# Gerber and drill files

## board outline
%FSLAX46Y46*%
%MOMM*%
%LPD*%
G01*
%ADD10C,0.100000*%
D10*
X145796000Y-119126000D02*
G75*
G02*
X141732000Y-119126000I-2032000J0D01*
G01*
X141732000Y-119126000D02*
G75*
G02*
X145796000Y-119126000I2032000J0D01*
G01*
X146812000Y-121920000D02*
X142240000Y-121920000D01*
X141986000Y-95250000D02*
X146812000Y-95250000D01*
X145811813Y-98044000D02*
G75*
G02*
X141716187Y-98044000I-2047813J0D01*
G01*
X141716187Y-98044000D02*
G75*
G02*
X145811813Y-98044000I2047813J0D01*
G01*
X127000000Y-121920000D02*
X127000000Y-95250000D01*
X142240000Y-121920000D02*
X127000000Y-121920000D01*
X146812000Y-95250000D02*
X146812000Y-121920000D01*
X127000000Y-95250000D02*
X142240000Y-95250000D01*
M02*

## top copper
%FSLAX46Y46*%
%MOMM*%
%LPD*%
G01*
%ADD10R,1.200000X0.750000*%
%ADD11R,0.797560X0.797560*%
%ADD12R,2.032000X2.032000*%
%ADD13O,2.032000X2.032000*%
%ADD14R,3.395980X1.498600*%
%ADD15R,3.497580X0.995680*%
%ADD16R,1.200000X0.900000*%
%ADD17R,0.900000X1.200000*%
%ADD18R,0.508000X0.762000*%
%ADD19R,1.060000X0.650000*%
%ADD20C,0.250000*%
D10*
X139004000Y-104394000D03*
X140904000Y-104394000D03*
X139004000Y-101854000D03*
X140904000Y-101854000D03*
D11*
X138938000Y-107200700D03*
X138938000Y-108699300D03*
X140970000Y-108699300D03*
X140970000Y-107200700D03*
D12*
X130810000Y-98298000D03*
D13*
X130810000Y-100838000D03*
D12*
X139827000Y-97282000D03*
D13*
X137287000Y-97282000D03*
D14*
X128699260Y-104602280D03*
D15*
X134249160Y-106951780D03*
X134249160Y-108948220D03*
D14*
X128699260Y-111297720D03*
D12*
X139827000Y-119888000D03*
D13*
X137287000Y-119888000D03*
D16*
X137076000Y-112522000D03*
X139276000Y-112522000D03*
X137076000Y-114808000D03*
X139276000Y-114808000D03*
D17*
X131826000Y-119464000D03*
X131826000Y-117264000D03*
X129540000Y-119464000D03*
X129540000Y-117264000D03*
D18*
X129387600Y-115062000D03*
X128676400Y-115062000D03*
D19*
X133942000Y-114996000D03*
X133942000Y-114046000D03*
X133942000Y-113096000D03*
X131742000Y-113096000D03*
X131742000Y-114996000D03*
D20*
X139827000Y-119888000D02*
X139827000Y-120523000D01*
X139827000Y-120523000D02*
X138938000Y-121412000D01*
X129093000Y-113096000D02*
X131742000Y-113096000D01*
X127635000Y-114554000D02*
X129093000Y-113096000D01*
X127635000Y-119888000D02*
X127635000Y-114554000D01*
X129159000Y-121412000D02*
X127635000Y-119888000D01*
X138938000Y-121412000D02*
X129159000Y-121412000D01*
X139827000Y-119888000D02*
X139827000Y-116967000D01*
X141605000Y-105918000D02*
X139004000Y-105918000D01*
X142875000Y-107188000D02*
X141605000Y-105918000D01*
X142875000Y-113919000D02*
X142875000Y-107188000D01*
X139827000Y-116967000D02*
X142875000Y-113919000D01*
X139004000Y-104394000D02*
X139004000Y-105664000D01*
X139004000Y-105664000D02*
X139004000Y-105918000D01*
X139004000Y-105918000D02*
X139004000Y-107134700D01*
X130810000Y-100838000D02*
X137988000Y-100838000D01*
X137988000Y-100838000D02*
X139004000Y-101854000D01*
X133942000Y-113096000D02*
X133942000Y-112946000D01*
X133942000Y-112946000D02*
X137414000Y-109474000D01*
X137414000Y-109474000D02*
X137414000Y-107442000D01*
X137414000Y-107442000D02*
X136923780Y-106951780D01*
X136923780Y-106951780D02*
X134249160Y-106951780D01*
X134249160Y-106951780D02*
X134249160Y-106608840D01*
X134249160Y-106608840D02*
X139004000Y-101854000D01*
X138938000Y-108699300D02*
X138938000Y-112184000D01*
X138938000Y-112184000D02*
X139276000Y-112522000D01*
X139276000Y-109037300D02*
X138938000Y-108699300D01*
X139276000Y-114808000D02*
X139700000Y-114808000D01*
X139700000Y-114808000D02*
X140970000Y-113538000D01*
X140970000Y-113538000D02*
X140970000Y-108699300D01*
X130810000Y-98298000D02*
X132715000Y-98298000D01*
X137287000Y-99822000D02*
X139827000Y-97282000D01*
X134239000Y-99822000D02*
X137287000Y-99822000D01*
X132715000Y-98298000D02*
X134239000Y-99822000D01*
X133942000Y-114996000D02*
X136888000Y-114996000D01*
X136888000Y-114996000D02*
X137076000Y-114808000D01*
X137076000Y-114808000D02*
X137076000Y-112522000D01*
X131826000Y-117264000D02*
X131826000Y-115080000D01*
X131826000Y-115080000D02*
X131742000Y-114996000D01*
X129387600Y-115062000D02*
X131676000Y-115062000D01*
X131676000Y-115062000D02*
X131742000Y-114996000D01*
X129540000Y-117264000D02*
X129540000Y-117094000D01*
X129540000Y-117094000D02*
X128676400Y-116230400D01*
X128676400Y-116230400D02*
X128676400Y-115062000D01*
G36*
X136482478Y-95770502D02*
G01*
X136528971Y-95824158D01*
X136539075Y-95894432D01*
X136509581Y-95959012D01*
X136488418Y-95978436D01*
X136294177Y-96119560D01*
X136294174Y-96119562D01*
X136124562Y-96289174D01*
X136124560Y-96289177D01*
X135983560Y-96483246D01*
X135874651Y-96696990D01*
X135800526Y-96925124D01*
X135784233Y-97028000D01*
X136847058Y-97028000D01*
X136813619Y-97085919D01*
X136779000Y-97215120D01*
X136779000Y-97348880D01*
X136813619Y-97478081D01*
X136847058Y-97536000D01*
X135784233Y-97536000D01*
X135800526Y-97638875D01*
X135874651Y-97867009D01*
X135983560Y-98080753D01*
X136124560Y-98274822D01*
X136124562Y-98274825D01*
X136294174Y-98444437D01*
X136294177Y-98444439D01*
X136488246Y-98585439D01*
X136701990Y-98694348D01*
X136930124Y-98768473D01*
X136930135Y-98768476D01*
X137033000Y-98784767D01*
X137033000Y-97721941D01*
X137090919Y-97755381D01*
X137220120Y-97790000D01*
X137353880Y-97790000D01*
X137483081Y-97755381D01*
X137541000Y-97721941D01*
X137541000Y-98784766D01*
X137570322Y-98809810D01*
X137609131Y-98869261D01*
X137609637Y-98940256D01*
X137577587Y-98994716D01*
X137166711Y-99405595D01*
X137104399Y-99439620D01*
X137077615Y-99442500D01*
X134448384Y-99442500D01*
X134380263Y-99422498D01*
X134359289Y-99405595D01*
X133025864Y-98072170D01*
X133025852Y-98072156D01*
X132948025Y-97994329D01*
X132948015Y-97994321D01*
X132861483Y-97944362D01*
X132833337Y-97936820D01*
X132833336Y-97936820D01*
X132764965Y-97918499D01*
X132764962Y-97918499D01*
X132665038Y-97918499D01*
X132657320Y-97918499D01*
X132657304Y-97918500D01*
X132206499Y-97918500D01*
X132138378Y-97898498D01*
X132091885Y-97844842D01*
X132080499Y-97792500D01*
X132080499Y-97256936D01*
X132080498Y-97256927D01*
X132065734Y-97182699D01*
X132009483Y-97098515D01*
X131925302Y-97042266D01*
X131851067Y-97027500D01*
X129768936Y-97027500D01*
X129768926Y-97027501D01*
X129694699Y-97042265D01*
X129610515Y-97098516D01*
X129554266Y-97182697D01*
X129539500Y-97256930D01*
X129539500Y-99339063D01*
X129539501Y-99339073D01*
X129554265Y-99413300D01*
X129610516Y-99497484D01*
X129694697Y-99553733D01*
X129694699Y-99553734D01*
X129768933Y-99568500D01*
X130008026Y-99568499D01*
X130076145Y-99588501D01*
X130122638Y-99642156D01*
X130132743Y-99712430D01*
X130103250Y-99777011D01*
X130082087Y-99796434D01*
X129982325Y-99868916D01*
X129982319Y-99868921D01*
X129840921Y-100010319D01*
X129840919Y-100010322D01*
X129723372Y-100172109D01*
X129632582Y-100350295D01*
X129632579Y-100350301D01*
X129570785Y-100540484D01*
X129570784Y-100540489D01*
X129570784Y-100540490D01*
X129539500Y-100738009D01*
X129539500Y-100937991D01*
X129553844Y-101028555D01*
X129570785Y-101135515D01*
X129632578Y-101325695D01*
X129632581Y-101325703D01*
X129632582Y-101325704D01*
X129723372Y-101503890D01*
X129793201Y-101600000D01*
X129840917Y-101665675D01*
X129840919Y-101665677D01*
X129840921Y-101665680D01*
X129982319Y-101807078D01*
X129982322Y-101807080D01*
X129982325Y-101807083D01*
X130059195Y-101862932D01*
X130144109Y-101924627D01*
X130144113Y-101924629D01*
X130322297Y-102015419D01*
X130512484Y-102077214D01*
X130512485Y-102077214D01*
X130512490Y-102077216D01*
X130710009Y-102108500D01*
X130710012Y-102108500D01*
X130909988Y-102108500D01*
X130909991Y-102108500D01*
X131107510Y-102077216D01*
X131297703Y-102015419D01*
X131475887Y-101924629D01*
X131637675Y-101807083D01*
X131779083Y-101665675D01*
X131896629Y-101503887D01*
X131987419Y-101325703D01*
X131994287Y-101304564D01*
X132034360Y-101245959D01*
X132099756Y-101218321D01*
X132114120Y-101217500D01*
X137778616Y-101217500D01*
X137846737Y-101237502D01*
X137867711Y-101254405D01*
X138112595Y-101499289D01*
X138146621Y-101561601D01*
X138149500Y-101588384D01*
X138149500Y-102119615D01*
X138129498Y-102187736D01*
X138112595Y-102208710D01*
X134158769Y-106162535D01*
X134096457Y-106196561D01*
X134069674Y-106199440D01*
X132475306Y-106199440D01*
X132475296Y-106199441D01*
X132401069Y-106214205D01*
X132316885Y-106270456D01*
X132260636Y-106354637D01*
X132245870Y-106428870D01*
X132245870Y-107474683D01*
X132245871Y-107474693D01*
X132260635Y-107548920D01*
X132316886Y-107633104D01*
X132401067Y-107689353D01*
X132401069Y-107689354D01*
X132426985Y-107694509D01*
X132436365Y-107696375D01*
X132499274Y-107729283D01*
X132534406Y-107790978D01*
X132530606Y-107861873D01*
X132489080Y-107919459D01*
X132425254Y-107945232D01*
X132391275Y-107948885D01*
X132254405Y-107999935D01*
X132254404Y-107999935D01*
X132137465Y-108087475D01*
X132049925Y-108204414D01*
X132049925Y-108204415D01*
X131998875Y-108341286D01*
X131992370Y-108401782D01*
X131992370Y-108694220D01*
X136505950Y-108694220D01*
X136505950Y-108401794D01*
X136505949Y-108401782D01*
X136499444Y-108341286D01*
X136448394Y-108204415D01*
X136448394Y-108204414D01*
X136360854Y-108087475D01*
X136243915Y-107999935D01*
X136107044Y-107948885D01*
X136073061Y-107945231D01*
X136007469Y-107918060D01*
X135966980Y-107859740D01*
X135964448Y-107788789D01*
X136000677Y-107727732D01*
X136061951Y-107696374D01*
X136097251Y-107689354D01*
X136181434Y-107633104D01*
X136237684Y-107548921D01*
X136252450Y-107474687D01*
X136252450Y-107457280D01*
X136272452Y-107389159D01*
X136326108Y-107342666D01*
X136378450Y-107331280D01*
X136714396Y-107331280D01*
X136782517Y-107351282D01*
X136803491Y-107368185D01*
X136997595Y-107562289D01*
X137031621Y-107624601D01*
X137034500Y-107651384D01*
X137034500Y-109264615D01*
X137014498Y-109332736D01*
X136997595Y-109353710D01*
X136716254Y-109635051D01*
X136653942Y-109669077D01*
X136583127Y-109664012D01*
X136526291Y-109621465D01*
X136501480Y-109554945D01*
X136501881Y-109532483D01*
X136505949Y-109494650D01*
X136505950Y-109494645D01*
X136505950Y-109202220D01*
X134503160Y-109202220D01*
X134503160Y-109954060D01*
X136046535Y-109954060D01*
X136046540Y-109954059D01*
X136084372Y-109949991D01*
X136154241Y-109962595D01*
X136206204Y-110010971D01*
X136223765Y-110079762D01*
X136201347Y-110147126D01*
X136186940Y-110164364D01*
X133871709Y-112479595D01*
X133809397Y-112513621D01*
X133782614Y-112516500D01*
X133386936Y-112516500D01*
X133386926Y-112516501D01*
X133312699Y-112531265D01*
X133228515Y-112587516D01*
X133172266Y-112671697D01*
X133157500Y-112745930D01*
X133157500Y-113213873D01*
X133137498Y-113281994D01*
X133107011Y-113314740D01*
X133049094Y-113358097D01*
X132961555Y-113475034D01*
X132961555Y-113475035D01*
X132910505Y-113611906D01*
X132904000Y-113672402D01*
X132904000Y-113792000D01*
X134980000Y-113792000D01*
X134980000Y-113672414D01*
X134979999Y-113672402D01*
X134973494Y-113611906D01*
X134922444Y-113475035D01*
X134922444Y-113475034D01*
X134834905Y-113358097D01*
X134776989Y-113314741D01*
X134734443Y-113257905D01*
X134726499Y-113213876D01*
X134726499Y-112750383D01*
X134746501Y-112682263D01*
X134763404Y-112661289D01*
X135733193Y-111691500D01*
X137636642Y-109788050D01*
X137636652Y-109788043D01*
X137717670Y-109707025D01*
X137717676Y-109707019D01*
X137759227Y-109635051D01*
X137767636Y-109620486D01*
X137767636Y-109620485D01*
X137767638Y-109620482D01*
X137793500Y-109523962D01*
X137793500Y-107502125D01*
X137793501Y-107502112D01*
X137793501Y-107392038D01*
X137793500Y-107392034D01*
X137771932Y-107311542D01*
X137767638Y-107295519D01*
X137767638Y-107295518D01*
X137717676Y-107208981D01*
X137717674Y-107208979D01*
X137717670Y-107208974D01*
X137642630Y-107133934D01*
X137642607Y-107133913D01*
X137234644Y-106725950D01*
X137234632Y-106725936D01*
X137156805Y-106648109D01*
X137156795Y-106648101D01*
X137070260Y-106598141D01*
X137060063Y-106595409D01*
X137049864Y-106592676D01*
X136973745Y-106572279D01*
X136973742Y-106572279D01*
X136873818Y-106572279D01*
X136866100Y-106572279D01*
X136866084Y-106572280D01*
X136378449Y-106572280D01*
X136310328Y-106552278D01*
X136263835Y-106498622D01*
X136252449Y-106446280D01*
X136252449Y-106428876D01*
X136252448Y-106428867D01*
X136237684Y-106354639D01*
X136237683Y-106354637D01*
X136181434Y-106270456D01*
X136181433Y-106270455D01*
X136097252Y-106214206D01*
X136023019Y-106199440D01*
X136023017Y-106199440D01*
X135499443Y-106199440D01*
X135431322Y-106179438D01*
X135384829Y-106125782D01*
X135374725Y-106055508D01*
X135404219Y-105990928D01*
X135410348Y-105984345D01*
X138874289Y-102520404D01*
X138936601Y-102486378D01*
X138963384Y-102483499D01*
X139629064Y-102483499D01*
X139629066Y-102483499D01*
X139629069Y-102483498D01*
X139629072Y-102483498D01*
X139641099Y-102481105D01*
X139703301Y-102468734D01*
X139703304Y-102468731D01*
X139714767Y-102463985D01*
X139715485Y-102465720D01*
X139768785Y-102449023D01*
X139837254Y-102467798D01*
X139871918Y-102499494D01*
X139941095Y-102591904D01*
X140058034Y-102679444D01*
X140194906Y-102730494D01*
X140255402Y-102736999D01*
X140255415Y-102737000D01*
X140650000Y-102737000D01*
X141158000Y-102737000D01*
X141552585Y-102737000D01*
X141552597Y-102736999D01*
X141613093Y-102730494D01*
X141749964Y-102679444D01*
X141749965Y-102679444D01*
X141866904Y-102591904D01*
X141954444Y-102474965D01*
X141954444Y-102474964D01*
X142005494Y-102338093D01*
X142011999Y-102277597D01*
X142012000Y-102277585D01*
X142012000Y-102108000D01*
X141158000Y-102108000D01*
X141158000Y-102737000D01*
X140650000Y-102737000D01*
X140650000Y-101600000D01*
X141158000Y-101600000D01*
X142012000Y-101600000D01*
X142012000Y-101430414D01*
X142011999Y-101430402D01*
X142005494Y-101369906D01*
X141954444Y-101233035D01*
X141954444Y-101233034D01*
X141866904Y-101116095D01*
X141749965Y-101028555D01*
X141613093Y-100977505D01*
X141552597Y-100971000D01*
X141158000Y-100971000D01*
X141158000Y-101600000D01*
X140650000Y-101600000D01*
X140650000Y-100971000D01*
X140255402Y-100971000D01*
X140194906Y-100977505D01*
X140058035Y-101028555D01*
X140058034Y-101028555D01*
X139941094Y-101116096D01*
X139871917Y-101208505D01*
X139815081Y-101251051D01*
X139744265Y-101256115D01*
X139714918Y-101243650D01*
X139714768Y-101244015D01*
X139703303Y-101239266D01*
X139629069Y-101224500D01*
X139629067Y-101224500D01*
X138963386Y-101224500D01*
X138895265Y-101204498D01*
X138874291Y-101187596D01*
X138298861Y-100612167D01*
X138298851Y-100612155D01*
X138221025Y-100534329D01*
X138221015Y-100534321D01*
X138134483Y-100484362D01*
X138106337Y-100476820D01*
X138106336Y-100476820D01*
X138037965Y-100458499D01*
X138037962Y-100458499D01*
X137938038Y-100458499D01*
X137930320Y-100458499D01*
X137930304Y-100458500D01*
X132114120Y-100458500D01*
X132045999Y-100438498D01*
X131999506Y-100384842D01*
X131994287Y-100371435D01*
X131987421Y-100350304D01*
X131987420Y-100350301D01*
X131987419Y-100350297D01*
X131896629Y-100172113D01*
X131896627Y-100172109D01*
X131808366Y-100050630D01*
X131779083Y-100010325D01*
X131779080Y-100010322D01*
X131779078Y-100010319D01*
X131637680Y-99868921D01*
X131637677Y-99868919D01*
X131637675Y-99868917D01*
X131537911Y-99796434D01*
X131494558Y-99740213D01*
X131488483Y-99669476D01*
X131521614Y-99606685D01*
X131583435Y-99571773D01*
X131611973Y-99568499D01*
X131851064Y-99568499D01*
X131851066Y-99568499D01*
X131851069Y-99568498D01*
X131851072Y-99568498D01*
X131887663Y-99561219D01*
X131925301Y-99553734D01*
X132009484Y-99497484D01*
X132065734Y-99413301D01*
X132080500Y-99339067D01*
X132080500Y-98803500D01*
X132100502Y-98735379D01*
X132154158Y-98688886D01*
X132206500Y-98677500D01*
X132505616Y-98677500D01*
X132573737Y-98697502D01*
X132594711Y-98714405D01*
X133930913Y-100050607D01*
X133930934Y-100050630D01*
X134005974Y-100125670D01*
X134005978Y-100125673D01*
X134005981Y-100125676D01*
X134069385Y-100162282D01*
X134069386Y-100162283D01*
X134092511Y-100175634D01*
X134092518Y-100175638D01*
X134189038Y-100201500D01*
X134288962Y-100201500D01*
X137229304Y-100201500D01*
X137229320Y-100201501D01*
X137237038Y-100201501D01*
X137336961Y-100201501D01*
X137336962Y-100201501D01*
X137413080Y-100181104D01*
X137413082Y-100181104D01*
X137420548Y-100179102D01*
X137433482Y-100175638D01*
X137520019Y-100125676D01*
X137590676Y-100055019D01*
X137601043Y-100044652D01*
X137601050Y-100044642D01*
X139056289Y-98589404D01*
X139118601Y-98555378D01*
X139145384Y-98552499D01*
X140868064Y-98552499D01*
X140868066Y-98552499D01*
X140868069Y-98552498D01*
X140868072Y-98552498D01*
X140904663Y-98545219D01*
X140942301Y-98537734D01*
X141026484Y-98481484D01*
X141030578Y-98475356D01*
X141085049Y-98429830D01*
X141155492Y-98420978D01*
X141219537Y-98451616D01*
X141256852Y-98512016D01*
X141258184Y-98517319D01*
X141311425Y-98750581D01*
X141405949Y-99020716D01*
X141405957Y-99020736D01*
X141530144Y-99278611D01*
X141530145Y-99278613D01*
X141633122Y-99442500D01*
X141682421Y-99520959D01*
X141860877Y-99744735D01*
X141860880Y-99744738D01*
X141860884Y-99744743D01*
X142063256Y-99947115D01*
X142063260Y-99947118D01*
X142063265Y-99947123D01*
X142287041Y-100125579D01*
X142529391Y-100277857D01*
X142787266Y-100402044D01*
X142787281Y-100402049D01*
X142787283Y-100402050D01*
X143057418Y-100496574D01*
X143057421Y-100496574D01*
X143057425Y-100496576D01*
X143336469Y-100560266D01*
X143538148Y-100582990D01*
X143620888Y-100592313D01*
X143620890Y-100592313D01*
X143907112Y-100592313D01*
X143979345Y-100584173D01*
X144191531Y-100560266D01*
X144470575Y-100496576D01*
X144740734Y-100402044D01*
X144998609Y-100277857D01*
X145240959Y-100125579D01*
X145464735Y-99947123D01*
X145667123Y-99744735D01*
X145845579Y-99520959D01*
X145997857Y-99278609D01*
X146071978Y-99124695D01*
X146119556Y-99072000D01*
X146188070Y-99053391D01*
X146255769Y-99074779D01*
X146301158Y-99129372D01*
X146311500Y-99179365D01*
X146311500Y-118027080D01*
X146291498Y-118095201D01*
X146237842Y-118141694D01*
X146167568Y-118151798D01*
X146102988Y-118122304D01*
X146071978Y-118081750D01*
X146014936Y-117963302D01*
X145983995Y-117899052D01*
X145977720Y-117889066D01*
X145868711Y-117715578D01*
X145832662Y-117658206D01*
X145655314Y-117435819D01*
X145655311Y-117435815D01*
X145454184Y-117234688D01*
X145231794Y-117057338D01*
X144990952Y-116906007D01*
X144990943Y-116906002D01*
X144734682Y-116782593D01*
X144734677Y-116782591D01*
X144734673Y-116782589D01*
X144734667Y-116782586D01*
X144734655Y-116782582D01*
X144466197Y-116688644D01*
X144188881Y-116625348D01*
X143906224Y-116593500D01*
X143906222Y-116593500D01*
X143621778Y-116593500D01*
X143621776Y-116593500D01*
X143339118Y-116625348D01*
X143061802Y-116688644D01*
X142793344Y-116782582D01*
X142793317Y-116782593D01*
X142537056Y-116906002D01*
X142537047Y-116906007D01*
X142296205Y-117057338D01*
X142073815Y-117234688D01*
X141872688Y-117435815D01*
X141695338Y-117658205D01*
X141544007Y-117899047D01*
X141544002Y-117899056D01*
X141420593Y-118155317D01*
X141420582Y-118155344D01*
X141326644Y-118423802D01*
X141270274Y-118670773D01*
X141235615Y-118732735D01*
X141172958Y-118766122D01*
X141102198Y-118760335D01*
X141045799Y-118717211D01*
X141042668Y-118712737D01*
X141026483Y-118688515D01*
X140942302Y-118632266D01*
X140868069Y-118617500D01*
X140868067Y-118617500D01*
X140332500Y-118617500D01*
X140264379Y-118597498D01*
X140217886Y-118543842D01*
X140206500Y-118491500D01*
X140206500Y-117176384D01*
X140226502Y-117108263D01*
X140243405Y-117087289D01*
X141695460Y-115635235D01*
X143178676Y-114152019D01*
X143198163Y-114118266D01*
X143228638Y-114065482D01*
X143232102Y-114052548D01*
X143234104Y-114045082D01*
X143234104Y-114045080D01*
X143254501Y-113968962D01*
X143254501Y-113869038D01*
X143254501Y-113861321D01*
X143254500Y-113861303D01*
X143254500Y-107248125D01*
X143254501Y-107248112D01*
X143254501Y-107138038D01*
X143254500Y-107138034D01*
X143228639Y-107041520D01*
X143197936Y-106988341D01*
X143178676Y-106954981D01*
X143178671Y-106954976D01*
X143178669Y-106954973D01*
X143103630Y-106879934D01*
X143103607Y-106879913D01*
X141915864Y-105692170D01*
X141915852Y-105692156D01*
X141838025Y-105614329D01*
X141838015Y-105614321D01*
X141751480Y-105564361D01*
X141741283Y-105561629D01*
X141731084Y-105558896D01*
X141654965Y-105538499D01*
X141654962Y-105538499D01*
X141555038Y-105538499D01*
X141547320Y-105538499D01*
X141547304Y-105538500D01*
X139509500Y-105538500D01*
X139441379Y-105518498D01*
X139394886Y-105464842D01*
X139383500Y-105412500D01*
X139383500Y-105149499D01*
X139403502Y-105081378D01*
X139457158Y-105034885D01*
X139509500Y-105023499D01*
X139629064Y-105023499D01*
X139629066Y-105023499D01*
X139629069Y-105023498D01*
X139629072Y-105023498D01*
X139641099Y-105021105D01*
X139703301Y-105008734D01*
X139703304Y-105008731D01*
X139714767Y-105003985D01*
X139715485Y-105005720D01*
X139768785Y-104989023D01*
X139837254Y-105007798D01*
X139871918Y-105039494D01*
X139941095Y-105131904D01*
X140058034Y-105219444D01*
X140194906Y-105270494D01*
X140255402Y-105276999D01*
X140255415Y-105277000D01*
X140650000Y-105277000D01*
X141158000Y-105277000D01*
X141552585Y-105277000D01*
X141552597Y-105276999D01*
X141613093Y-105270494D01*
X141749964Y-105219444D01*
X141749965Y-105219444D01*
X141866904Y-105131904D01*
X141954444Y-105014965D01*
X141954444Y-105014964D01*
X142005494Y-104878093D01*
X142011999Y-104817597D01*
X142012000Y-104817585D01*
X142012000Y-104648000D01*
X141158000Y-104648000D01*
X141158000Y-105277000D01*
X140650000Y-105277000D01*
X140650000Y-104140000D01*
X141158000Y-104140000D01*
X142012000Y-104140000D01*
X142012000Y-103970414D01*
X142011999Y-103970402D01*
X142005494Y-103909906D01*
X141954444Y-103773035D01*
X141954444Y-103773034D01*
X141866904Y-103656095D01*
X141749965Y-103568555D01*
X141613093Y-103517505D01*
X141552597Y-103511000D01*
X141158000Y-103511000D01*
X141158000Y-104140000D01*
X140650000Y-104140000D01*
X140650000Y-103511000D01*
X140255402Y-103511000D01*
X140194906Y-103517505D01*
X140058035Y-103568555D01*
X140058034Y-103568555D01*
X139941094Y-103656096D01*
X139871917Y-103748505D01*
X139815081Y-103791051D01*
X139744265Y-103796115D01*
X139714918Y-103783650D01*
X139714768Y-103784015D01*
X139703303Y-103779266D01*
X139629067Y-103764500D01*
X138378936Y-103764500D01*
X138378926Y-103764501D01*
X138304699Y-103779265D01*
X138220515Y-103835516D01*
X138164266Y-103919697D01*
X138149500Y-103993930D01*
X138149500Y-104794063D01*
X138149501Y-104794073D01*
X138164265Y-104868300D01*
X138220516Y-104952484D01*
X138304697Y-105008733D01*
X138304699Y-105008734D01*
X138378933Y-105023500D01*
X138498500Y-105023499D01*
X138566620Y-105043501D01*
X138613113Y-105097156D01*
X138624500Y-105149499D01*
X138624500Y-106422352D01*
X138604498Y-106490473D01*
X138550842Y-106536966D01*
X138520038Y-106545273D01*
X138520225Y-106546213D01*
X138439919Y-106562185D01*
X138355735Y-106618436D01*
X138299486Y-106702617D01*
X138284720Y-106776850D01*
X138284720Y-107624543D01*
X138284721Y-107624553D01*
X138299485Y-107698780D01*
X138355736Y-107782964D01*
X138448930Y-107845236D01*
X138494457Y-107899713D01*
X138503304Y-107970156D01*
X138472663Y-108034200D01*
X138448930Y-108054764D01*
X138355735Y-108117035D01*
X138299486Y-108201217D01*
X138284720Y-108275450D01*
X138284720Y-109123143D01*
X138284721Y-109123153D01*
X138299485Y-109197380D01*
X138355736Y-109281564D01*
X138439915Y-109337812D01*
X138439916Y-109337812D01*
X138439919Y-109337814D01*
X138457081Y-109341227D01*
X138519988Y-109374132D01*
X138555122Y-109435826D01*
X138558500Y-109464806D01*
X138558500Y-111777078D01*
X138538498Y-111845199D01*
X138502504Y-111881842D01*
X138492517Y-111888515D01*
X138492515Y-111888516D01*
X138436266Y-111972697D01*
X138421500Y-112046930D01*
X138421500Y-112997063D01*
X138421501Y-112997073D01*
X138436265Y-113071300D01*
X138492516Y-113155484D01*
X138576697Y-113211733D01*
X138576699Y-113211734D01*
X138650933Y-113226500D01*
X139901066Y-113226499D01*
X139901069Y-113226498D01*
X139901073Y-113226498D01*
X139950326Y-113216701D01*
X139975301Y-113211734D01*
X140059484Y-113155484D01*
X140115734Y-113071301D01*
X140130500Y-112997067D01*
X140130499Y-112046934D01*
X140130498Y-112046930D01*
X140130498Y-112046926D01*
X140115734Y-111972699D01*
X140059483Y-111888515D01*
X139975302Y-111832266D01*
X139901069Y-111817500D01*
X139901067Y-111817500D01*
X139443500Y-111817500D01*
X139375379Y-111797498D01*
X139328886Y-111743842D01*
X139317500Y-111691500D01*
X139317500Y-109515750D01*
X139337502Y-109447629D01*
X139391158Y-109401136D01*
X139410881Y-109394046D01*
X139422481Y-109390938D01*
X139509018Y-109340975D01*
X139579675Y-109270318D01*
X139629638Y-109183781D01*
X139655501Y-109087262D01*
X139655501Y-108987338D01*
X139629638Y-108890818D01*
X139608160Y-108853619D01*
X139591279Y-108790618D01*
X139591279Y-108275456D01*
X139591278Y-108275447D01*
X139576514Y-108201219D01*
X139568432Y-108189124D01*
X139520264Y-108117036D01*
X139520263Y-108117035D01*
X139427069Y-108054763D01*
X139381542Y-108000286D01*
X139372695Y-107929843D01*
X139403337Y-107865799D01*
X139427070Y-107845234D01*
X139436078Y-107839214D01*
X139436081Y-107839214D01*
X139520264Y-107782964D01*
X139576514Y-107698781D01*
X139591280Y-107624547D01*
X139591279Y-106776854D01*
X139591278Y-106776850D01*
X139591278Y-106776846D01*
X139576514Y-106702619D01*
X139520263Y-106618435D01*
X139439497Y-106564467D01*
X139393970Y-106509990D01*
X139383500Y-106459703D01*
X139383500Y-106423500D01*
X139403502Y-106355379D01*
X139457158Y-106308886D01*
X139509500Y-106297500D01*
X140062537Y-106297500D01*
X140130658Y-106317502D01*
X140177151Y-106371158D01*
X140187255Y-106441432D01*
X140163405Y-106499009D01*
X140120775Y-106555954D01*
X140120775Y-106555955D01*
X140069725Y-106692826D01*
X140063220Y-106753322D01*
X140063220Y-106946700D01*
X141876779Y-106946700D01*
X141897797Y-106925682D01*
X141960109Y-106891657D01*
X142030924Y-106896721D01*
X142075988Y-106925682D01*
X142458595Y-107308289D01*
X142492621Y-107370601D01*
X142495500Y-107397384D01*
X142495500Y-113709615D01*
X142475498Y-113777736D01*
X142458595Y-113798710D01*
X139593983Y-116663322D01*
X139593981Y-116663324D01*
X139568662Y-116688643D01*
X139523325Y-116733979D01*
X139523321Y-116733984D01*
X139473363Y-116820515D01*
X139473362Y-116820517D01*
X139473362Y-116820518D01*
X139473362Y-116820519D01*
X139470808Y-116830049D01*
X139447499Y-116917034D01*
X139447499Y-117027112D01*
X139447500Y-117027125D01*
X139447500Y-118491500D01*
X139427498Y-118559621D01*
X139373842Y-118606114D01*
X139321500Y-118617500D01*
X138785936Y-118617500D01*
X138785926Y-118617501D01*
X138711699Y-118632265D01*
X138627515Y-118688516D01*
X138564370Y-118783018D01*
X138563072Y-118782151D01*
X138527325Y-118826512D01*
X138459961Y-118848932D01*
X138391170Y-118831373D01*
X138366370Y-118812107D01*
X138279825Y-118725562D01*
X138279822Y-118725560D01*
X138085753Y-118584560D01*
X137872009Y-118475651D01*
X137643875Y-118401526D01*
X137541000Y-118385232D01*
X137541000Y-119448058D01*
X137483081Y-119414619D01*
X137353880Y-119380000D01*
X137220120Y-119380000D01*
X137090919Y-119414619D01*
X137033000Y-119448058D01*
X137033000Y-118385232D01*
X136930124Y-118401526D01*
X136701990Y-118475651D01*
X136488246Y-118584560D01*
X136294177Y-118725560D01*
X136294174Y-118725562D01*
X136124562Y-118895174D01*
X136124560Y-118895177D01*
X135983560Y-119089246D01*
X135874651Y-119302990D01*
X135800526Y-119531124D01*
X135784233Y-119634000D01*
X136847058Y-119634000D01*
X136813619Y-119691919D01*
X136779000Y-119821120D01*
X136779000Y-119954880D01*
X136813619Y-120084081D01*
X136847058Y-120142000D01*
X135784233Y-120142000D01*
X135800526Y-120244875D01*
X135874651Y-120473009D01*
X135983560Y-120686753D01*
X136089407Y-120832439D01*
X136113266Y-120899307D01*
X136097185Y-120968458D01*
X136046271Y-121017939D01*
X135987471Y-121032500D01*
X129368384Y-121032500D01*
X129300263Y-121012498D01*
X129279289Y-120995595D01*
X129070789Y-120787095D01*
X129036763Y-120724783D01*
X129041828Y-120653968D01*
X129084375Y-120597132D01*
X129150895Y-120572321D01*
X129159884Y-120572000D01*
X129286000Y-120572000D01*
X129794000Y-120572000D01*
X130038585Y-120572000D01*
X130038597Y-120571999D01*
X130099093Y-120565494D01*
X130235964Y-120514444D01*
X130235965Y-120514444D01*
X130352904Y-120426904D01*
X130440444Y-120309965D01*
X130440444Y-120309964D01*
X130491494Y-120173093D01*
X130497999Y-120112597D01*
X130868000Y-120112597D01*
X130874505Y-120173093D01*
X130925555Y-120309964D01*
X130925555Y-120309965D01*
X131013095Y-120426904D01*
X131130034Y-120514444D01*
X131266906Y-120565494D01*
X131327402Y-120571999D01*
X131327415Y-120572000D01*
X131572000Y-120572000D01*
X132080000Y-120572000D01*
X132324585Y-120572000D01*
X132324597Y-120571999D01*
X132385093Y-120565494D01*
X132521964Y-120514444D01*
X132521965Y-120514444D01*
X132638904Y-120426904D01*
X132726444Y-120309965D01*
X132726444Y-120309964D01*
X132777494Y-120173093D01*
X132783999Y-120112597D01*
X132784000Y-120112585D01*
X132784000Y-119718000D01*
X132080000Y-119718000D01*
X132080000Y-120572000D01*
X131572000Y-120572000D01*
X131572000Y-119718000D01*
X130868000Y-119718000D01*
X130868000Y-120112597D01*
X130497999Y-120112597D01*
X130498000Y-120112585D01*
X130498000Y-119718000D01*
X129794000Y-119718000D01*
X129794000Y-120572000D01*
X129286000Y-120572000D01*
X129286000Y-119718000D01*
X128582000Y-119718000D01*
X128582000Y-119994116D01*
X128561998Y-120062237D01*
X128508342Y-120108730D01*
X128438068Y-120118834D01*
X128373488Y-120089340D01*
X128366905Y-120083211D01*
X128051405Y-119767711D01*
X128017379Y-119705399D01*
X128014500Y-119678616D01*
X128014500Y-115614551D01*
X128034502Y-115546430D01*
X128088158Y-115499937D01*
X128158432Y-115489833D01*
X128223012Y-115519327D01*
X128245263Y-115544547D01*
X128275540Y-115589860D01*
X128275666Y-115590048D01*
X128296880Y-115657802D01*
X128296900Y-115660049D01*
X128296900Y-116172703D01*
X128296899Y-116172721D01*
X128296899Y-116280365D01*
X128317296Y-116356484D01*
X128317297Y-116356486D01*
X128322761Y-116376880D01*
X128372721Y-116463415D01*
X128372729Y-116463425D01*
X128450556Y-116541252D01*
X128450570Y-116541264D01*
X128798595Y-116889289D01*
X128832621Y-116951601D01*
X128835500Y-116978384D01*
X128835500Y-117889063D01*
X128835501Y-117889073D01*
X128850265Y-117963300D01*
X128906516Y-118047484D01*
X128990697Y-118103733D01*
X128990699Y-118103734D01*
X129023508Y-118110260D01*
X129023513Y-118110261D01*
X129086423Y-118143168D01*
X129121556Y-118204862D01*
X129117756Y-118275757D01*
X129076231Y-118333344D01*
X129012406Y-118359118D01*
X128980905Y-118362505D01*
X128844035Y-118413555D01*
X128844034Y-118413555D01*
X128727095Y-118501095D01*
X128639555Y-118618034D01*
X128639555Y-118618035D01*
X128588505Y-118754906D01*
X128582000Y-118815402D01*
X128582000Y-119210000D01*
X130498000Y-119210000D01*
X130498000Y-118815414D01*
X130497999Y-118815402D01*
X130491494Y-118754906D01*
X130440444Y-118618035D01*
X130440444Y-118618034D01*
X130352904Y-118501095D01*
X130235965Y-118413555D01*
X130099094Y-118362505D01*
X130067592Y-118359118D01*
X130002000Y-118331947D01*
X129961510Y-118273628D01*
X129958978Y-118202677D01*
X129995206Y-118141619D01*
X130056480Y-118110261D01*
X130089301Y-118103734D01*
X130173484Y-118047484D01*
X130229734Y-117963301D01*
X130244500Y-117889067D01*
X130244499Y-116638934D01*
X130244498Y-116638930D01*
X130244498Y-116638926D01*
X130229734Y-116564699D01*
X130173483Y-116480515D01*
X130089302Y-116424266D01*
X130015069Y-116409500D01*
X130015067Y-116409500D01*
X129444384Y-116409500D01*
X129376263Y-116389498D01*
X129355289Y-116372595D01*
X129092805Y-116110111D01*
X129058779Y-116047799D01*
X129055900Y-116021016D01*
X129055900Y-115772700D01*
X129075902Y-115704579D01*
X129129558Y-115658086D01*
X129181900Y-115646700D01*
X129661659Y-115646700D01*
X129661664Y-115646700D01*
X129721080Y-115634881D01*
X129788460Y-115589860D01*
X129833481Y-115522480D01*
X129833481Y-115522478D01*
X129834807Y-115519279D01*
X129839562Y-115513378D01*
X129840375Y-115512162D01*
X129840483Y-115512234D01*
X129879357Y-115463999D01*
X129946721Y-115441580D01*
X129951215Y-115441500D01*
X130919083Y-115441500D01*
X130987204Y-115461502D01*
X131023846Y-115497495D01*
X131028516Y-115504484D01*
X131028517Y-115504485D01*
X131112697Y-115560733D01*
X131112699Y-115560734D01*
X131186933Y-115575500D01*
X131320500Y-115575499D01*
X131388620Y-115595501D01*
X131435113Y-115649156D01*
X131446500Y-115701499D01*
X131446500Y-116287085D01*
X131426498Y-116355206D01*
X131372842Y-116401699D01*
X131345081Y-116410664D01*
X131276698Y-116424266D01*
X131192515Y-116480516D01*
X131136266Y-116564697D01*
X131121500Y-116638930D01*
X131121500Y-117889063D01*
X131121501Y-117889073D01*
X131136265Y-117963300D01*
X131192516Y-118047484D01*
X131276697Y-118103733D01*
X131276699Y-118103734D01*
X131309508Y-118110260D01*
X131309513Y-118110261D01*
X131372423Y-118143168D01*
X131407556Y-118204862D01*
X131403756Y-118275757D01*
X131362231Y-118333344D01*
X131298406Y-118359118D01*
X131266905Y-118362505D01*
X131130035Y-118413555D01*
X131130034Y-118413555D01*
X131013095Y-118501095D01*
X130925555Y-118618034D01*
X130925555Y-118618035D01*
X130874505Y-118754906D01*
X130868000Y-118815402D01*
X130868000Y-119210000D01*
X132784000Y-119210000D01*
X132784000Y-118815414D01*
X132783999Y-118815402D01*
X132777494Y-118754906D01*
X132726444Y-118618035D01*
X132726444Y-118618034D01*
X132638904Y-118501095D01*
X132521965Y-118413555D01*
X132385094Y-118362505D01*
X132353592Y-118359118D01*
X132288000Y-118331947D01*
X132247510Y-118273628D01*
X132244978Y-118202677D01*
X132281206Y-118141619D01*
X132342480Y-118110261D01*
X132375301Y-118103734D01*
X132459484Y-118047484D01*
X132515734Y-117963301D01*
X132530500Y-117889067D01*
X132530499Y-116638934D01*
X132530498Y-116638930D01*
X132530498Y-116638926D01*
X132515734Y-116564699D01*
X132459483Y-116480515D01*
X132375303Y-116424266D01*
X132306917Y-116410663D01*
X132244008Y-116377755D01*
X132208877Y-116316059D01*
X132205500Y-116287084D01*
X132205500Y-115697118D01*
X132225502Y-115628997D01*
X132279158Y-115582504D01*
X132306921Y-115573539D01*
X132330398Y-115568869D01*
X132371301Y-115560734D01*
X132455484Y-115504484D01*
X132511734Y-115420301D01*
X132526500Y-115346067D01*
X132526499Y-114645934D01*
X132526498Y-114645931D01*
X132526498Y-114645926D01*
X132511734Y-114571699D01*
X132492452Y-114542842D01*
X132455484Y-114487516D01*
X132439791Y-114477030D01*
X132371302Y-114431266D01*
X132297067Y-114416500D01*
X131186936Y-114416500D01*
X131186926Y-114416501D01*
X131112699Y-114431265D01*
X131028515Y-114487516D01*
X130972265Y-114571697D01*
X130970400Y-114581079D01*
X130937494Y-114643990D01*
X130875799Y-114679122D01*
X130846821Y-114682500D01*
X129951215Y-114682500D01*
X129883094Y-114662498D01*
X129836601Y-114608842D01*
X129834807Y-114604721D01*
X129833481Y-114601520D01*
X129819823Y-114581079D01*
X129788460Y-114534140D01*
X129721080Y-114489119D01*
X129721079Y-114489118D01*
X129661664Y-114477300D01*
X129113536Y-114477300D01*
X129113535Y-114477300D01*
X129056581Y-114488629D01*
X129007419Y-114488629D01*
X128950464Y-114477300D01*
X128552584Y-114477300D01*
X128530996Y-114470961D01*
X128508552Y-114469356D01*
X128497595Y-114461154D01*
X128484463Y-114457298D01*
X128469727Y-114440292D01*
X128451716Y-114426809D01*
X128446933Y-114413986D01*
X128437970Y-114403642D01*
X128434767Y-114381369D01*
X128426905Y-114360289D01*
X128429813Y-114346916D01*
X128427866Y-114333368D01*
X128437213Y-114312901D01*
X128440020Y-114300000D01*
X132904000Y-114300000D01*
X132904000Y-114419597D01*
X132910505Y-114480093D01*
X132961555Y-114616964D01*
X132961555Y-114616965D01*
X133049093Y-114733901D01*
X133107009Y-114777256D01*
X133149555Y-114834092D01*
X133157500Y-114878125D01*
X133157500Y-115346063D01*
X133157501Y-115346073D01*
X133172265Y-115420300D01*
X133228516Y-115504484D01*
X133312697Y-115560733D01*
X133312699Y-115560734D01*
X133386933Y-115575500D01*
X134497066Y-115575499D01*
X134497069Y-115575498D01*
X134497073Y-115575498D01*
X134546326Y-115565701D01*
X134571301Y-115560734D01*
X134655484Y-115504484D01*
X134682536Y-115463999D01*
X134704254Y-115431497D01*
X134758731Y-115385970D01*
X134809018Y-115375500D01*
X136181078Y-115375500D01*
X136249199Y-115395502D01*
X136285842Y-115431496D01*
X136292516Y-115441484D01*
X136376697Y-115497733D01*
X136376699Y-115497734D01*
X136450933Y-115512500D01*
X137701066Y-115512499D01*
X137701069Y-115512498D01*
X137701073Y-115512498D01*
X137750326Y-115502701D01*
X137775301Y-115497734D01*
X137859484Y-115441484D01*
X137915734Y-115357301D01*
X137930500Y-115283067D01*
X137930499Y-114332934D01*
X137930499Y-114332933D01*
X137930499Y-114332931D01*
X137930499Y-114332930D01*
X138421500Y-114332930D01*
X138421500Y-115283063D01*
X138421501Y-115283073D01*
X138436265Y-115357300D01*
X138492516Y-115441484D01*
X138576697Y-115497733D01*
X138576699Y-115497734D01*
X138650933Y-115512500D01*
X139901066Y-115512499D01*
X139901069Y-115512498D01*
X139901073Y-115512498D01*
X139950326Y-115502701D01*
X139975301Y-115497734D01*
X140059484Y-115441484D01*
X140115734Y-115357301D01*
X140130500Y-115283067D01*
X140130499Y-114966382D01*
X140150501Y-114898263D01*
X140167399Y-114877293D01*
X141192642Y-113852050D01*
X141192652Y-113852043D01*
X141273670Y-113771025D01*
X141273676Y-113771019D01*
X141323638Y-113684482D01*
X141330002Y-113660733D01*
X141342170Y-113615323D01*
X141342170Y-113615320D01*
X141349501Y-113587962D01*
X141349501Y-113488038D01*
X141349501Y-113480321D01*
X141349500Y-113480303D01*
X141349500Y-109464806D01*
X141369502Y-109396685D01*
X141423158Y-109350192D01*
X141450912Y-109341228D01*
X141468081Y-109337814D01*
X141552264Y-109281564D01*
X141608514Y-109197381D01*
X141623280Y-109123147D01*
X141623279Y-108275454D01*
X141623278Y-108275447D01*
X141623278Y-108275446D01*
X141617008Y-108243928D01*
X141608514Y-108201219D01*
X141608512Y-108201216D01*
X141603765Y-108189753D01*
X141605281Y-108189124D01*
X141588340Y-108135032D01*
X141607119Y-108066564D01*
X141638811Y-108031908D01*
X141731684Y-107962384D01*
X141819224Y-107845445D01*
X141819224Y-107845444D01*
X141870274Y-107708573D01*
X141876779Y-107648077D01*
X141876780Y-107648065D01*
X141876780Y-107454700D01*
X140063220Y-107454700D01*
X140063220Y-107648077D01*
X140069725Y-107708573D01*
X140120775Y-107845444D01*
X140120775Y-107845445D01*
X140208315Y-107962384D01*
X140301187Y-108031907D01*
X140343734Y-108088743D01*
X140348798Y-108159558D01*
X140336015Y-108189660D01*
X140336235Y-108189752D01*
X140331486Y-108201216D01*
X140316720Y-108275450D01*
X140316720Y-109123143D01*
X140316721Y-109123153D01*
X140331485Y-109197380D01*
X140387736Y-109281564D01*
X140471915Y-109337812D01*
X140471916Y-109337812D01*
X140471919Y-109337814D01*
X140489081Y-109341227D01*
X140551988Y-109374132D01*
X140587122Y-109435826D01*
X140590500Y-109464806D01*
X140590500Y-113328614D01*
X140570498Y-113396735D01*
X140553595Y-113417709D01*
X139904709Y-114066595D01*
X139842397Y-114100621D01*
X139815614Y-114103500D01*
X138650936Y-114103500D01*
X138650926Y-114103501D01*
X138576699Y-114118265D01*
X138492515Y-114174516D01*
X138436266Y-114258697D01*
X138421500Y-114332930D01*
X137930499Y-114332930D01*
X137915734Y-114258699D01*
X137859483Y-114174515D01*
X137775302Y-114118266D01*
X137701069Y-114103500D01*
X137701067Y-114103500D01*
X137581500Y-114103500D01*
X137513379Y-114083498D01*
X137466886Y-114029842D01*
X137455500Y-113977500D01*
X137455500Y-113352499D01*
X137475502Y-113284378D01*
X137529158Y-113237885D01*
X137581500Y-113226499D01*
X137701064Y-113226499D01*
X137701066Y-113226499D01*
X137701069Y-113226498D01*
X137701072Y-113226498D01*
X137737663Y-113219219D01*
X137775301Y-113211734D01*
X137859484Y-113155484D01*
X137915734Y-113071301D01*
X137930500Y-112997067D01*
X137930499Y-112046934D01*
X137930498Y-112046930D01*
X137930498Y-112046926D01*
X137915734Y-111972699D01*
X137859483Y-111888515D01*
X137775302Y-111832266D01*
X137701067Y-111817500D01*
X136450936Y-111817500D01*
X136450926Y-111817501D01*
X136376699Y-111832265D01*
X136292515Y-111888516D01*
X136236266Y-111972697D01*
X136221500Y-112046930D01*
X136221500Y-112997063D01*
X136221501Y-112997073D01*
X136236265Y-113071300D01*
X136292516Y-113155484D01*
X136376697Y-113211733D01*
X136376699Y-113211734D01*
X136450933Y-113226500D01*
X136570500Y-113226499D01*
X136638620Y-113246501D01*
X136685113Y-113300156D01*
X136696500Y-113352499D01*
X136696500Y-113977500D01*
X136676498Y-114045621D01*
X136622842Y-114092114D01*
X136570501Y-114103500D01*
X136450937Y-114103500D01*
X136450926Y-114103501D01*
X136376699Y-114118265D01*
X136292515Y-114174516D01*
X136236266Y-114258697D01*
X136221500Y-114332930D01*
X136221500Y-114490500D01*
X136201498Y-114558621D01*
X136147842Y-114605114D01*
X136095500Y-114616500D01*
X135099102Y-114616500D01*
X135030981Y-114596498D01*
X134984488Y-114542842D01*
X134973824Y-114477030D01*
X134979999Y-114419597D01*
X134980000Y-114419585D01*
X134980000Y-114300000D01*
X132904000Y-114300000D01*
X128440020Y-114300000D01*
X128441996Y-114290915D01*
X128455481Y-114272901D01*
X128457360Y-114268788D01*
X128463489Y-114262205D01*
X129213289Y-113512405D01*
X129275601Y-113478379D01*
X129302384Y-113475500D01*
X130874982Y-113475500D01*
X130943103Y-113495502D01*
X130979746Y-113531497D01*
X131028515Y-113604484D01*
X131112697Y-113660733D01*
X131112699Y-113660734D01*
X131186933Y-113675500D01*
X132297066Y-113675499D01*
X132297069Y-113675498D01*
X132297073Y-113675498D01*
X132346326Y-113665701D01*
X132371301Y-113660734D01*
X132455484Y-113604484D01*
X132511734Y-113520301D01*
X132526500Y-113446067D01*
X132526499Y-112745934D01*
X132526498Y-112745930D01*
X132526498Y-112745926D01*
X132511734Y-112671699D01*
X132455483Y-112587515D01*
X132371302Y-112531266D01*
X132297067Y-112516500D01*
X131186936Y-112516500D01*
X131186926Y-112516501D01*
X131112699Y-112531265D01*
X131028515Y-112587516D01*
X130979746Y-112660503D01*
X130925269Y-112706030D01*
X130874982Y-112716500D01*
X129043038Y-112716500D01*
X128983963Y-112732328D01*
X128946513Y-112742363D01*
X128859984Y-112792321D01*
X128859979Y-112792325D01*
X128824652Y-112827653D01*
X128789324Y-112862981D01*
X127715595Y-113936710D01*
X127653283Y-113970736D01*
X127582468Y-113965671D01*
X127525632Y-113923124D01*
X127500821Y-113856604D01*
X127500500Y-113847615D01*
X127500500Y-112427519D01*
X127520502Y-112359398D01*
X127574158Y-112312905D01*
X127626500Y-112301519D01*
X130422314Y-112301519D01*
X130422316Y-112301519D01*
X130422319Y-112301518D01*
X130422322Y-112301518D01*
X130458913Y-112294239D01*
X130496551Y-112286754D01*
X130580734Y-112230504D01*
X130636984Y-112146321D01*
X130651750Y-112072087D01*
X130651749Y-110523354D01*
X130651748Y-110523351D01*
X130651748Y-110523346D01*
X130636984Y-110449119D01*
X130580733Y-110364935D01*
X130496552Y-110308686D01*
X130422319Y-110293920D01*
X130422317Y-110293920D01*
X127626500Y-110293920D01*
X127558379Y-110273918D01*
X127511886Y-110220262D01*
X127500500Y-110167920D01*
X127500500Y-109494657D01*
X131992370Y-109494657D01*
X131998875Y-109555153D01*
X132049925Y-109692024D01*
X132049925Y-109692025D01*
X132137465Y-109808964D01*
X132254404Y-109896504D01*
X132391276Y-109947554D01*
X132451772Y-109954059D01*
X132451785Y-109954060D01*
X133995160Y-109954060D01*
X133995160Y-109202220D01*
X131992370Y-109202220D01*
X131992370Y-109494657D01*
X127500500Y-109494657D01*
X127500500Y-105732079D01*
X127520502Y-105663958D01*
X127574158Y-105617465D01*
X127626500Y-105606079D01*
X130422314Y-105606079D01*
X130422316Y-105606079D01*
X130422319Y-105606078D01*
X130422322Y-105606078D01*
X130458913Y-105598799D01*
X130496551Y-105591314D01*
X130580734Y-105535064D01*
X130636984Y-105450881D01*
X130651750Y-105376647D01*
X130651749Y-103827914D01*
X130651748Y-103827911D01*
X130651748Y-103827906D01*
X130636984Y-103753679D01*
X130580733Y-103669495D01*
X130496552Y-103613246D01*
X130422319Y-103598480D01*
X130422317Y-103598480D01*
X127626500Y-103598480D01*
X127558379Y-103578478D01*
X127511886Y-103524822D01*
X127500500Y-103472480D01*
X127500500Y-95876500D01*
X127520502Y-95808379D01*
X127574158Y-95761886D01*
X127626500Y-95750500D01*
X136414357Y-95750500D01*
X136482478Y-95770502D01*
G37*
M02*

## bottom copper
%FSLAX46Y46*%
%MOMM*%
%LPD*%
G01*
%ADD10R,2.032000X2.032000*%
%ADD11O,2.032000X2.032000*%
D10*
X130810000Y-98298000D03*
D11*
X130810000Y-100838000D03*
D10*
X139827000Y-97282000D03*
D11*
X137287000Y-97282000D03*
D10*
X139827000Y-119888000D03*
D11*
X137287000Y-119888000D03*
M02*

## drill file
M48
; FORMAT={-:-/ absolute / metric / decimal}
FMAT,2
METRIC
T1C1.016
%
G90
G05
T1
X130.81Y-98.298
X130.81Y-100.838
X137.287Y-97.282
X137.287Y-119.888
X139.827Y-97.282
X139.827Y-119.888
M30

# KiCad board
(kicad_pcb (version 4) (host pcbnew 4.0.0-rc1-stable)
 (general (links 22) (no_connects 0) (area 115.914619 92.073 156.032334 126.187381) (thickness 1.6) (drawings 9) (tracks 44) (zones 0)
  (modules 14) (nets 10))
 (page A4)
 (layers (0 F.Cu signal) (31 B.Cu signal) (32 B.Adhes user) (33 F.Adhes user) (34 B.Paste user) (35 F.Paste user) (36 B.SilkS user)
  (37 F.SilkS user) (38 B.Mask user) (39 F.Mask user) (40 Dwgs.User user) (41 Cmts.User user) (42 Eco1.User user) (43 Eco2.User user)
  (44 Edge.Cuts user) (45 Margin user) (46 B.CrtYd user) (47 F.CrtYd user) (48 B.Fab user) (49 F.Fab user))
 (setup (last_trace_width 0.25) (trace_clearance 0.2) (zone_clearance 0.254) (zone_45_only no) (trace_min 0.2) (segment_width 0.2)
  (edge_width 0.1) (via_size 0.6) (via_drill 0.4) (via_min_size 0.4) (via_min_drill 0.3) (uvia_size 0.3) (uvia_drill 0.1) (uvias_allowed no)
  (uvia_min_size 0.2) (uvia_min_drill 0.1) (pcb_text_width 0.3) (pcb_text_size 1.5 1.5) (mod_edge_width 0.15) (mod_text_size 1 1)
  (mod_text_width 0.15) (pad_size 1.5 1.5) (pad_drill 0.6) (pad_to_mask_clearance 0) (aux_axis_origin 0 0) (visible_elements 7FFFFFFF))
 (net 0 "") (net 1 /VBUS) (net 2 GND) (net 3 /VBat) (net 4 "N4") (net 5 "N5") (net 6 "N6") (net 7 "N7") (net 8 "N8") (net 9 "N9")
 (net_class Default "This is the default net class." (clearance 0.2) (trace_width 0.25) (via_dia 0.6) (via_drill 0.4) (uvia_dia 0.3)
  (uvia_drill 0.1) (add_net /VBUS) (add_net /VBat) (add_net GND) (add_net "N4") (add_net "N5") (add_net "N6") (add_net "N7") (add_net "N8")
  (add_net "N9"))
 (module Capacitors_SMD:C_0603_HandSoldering (layer F.Cu) (at 139.954 104.394)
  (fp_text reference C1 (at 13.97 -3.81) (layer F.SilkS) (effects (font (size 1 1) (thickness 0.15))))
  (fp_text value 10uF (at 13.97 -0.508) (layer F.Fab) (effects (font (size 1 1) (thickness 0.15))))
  (pad 1 smd rect (at -0.95 0) (size 1.2 0.75) (layers F.Cu F.Paste F.Mask) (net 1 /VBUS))
  (pad 2 smd rect (at 0.95 0) (size 1.2 0.75) (layers F.Cu F.Paste F.Mask) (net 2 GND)))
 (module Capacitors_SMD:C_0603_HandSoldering (layer F.Cu) (at 139.954 101.854)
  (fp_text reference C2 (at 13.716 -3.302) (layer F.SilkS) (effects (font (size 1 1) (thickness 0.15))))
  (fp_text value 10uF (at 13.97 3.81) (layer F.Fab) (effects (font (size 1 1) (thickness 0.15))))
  (pad 1 smd rect (at -0.95 0) (size 1.2 0.75) (layers F.Cu F.Paste F.Mask) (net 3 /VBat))
  (pad 2 smd rect (at 0.95 0) (size 1.2 0.75) (layers F.Cu F.Paste F.Mask) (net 2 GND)))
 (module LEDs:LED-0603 (layer F.Cu) (at 138.938 107.95 90)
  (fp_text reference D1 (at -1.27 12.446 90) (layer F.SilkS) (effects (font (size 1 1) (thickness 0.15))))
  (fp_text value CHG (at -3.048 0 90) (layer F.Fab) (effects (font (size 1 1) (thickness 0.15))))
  (pad 2 smd rect (at 0.7493 0 270) (size 0.79756 0.79756) (layers F.Cu F.Paste F.Mask) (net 1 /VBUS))
  (pad 1 smd rect (at -0.7493 0 270) (size 0.79756 0.79756) (layers F.Cu F.Paste F.Mask) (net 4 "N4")))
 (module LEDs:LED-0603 (layer F.Cu) (at 140.97 107.95 270)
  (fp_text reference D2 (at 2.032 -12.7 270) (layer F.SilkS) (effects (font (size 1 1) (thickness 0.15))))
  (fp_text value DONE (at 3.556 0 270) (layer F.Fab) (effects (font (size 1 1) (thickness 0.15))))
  (pad 2 smd rect (at 0.7493 0 90) (size 0.79756 0.79756) (layers F.Cu F.Paste F.Mask) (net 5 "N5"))
  (pad 1 smd rect (at -0.7493 0 90) (size 0.79756 0.79756) (layers F.Cu F.Paste F.Mask) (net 2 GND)))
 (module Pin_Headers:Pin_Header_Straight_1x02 (layer F.Cu) (at 130.81 98.298)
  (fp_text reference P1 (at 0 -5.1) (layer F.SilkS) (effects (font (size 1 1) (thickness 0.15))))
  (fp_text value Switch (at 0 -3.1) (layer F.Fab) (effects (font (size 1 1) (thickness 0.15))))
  (pad 1 thru_hole rect (at 0 0) (size 2.032 2.032) (drill 1.016) (layers *.Cu *.Mask F.SilkS) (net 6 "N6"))
  (pad 2 thru_hole oval (at 0 2.54) (size 2.032 2.032) (drill 1.016) (layers *.Cu *.Mask F.SilkS) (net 3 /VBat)))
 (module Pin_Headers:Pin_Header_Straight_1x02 (layer F.Cu) (at 139.827 97.282 270)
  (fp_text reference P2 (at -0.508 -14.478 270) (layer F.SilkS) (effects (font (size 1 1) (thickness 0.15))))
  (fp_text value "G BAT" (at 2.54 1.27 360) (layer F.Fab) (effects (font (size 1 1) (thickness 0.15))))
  (pad 1 thru_hole rect (at 0 0 270) (size 2.032 2.032) (drill 1.016) (layers *.Cu *.Mask F.SilkS) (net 6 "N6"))
  (pad 2 thru_hole oval (at 0 2.54 270) (size 2.032 2.032) (drill 1.016) (layers *.Cu *.Mask F.SilkS) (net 2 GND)))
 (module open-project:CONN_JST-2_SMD (layer F.Cu) (at 127 107.95 270)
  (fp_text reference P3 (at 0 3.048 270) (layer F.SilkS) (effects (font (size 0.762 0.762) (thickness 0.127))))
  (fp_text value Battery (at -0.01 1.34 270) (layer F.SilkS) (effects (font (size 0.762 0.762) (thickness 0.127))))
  (pad "" smd rect (at -3.34772 -1.69926 270) (size 1.4986 3.39598) (layers F.Cu F.Paste F.Mask))
  (pad 1 smd rect (at -0.99822 -7.24916 270) (size 0.99568 3.49758) (layers F.Cu F.Paste F.Mask) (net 3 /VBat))
  (pad 2 smd rect (at 0.99822 -7.24916 270) (size 0.99568 3.49758) (layers F.Cu F.Paste F.Mask) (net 2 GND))
  (pad "" smd rect (at 3.34772 -1.69926 270) (size 1.4986 3.39598) (layers F.Cu F.Paste F.Mask)))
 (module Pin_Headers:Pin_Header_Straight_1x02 (layer F.Cu) (at 139.827 119.888 270)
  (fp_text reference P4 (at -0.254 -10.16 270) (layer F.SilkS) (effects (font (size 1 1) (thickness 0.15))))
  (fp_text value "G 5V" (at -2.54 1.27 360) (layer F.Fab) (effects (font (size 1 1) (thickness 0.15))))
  (pad 1 thru_hole rect (at 0 0 270) (size 2.032 2.032) (drill 1.016) (layers *.Cu *.Mask F.SilkS) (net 1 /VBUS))
  (pad 2 thru_hole oval (at 0 2.54 270) (size 2.032 2.032) (drill 1.016) (layers *.Cu *.Mask F.SilkS) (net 2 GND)))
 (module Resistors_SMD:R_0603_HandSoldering (layer F.Cu) (at 138.176 112.522)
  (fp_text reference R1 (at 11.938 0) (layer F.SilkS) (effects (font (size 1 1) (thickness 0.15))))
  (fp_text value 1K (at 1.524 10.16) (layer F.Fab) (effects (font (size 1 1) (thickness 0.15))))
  (pad 1 smd rect (at -1.1 0) (size 1.2 0.9) (layers F.Cu F.Paste F.Mask) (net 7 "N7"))
  (pad 2 smd rect (at 1.1 0) (size 1.2 0.9) (layers F.Cu F.Paste F.Mask) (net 4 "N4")))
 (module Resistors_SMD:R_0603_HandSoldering (layer F.Cu) (at 138.176 114.808)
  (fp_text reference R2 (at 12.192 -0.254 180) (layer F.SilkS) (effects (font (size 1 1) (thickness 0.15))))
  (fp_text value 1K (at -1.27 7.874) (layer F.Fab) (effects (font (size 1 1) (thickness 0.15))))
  (pad 1 smd rect (at -1.1 0) (size 1.2 0.9) (layers F.Cu F.Paste F.Mask) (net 7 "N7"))
  (pad 2 smd rect (at 1.1 0) (size 1.2 0.9) (layers F.Cu F.Paste F.Mask) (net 5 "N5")))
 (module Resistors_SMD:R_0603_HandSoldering (layer F.Cu) (at 131.826 118.364 90)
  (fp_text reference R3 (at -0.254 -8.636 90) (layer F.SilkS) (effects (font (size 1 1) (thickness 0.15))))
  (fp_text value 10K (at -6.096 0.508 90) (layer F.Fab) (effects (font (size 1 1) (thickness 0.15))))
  (pad 1 smd rect (at -1.1 0 90) (size 1.2 0.9) (layers F.Cu F.Paste F.Mask) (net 2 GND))
  (pad 2 smd rect (at 1.1 0 90) (size 1.2 0.9) (layers F.Cu F.Paste F.Mask) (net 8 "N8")))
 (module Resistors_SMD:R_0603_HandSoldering (layer F.Cu) (at 129.54 118.364 90)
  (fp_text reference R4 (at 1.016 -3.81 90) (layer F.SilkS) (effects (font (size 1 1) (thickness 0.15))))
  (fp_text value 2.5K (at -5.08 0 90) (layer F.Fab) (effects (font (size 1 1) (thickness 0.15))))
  (pad 1 smd rect (at -1.1 0 90) (size 1.2 0.9) (layers F.Cu F.Paste F.Mask) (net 2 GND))
  (pad 2 smd rect (at 1.1 0 90) (size 1.2 0.9) (layers F.Cu F.Paste F.Mask) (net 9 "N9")))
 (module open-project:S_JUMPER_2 (layer F.Cu) (at 129.032 115.062 180)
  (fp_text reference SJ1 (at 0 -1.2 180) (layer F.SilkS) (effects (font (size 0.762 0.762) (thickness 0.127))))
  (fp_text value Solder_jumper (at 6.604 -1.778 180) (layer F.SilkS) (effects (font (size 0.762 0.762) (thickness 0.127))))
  (pad 1 smd rect (at -0.3556 0 180) (size 0.508 0.762) (layers F.Cu F.Paste F.Mask) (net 8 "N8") (clearance 0.2032))
  (pad 2 smd rect (at 0.3556 0 180) (size 0.508 0.762) (layers F.Cu F.Paste F.Mask) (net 9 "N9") (clearance 0.2032)))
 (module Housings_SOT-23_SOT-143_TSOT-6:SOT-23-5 (layer F.Cu) (at 132.842 114.046 180)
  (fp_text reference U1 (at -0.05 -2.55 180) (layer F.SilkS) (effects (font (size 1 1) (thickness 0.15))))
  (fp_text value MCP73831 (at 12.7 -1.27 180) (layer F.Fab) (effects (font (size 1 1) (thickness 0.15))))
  (pad 1 smd rect (at -1.1 -0.95 180) (size 1.06 0.65) (layers F.Cu F.Paste F.Mask) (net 7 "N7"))
  (pad 2 smd rect (at -1.1 0 180) (size 1.06 0.65) (layers F.Cu F.Paste F.Mask) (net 2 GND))
  (pad 3 smd rect (at -1.1 0.95 180) (size 1.06 0.65) (layers F.Cu F.Paste F.Mask) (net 3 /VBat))
  (pad 4 smd rect (at 1.1 0.95 180) (size 1.06 0.65) (layers F.Cu F.Paste F.Mask) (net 1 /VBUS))
  (pad 5 smd rect (at 1.1 -0.95 180) (size 1.06 0.65) (layers F.Cu F.Paste F.Mask) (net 8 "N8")))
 (gr_circle (center 143.764 119.126) (end 145.796 119.126) (layer Edge.Cuts) (width 0.1))
 (gr_line (start 146.812 121.92) (end 142.24 121.92) (angle 90) (layer Edge.Cuts) (width 0.1))
 (gr_line (start 141.986 95.25) (end 146.812 95.25) (angle 90) (layer Edge.Cuts) (width 0.1))
 (gr_circle (center 143.764 98.044) (end 145.796 97.79) (layer Edge.Cuts) (width 0.1))
 (gr_line (start 127 121.92) (end 127 95.25) (angle 90) (layer Edge.Cuts) (width 0.1))
 (gr_line (start 142.24 121.92) (end 127 121.92) (angle 90) (layer Edge.Cuts) (width 0.1))
 (gr_line (start 146.812 95.25) (end 146.812 121.92) (angle 90) (layer Edge.Cuts) (width 0.1))
 (gr_line (start 127 95.25) (end 142.24 95.25) (angle 90) (layer Edge.Cuts) (width 0.1))
 (segment (start 139.827 119.888) (end 139.827 120.523) (width 0.25) (layer F.Cu) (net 1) (status C00000))
 (segment (start 139.827 120.523) (end 138.938 121.412) (width 0.25) (layer F.Cu) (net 1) (status 400000))
 (segment (start 129.093 113.096) (end 131.742 113.096) (width 0.25) (layer F.Cu) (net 1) (status 800000))
 (segment (start 127.635 114.554) (end 129.093 113.096) (width 0.25) (layer F.Cu) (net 1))
 (segment (start 127.635 119.888) (end 127.635 114.554) (width 0.25) (layer F.Cu) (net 1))
 (segment (start 129.159 121.412) (end 127.635 119.888) (width 0.25) (layer F.Cu) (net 1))
 (segment (start 138.938 121.412) (end 129.159 121.412) (width 0.25) (layer F.Cu) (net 1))
 (segment (start 139.827 119.888) (end 139.827 116.967) (width 0.25) (layer F.Cu) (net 1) (status 400000))
 (segment (start 141.605 105.918) (end 139.004 105.918) (width 0.25) (layer F.Cu) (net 1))
 (segment (start 142.875 107.188) (end 141.605 105.918) (width 0.25) (layer F.Cu) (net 1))
 (segment (start 142.875 113.919) (end 142.875 107.188) (width 0.25) (layer F.Cu) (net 1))
 (segment (start 139.827 116.967) (end 142.875 113.919) (width 0.25) (layer F.Cu) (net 1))
 (segment (start 139.004 104.394) (end 139.004 105.664) (width 0.25) (layer F.Cu) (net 1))
 (segment (start 139.004 105.664) (end 139.004 105.918) (width 0.25) (layer F.Cu) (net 1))
 (segment (start 139.004 105.918) (end 139.004 107.1347) (width 0.25) (layer F.Cu) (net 1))
 (segment (start 130.81 100.838) (end 137.988 100.838) (width 0.25) (layer F.Cu) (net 3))
 (segment (start 137.988 100.838) (end 139.004 101.854) (width 0.25) (layer F.Cu) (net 3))
 (segment (start 133.942 113.096) (end 133.942 112.946) (width 0.25) (layer F.Cu) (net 3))
 (segment (start 133.942 112.946) (end 137.414 109.474) (width 0.25) (layer F.Cu) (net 3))
 (segment (start 137.414 109.474) (end 137.414 107.442) (width 0.25) (layer F.Cu) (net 3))
 (segment (start 137.414 107.442) (end 136.92378 106.95178) (width 0.25) (layer F.Cu) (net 3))
 (segment (start 136.92378 106.95178) (end 134.24916 106.95178) (width 0.25) (layer F.Cu) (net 3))
 (segment (start 134.24916 106.95178) (end 134.24916 106.60884) (width 0.25) (layer F.Cu) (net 3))
 (segment (start 134.24916 106.60884) (end 139.004 101.854) (width 0.25) (layer F.Cu) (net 3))
 (segment (start 138.938 108.6993) (end 138.938 112.184) (width 0.25) (layer F.Cu) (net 4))
 (segment (start 138.938 112.184) (end 139.276 112.522) (width 0.25) (layer F.Cu) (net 4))
 (segment (start 139.276 109.0373) (end 138.938 108.6993) (width 0.25) (layer F.Cu) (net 4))
 (segment (start 139.276 114.808) (end 139.7 114.808) (width 0.25) (layer F.Cu) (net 5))
 (segment (start 139.7 114.808) (end 140.97 113.538) (width 0.25) (layer F.Cu) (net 5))
 (segment (start 140.97 113.538) (end 140.97 108.6993) (width 0.25) (layer F.Cu) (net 5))
 (segment (start 130.81 98.298) (end 132.715 98.298) (width 0.25) (layer F.Cu) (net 6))
 (segment (start 137.287 99.822) (end 139.827 97.282) (width 0.25) (layer F.Cu) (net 6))
 (segment (start 134.239 99.822) (end 137.287 99.822) (width 0.25) (layer F.Cu) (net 6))
 (segment (start 132.715 98.298) (end 134.239 99.822) (width 0.25) (layer F.Cu) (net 6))
 (segment (start 133.942 114.996) (end 136.888 114.996) (width 0.25) (layer F.Cu) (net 7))
 (segment (start 136.888 114.996) (end 137.076 114.808) (width 0.25) (layer F.Cu) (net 7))
 (segment (start 137.076 114.808) (end 137.076 112.522) (width 0.25) (layer F.Cu) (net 7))
 (segment (start 131.826 117.264) (end 131.826 115.08) (width 0.25) (layer F.Cu) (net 8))
 (segment (start 131.826 115.08) (end 131.742 114.996) (width 0.25) (layer F.Cu) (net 8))
 (segment (start 129.3876 115.062) (end 131.676 115.062) (width 0.25) (layer F.Cu) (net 8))
 (segment (start 131.676 115.062) (end 131.742 114.996) (width 0.25) (layer F.Cu) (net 8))
 (segment (start 129.54 117.264) (end 129.54 117.094) (width 0.25) (layer F.Cu) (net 9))
 (segment (start 129.54 117.094) (end 128.6764 116.2304) (width 0.25) (layer F.Cu) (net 9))
 (segment (start 128.6764 116.2304) (end 128.6764 115.062) (width 0.25) (layer F.Cu) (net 9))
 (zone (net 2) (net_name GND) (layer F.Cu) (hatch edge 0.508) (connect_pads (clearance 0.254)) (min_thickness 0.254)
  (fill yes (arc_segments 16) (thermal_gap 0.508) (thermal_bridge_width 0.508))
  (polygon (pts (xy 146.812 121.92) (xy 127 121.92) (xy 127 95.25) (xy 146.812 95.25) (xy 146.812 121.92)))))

